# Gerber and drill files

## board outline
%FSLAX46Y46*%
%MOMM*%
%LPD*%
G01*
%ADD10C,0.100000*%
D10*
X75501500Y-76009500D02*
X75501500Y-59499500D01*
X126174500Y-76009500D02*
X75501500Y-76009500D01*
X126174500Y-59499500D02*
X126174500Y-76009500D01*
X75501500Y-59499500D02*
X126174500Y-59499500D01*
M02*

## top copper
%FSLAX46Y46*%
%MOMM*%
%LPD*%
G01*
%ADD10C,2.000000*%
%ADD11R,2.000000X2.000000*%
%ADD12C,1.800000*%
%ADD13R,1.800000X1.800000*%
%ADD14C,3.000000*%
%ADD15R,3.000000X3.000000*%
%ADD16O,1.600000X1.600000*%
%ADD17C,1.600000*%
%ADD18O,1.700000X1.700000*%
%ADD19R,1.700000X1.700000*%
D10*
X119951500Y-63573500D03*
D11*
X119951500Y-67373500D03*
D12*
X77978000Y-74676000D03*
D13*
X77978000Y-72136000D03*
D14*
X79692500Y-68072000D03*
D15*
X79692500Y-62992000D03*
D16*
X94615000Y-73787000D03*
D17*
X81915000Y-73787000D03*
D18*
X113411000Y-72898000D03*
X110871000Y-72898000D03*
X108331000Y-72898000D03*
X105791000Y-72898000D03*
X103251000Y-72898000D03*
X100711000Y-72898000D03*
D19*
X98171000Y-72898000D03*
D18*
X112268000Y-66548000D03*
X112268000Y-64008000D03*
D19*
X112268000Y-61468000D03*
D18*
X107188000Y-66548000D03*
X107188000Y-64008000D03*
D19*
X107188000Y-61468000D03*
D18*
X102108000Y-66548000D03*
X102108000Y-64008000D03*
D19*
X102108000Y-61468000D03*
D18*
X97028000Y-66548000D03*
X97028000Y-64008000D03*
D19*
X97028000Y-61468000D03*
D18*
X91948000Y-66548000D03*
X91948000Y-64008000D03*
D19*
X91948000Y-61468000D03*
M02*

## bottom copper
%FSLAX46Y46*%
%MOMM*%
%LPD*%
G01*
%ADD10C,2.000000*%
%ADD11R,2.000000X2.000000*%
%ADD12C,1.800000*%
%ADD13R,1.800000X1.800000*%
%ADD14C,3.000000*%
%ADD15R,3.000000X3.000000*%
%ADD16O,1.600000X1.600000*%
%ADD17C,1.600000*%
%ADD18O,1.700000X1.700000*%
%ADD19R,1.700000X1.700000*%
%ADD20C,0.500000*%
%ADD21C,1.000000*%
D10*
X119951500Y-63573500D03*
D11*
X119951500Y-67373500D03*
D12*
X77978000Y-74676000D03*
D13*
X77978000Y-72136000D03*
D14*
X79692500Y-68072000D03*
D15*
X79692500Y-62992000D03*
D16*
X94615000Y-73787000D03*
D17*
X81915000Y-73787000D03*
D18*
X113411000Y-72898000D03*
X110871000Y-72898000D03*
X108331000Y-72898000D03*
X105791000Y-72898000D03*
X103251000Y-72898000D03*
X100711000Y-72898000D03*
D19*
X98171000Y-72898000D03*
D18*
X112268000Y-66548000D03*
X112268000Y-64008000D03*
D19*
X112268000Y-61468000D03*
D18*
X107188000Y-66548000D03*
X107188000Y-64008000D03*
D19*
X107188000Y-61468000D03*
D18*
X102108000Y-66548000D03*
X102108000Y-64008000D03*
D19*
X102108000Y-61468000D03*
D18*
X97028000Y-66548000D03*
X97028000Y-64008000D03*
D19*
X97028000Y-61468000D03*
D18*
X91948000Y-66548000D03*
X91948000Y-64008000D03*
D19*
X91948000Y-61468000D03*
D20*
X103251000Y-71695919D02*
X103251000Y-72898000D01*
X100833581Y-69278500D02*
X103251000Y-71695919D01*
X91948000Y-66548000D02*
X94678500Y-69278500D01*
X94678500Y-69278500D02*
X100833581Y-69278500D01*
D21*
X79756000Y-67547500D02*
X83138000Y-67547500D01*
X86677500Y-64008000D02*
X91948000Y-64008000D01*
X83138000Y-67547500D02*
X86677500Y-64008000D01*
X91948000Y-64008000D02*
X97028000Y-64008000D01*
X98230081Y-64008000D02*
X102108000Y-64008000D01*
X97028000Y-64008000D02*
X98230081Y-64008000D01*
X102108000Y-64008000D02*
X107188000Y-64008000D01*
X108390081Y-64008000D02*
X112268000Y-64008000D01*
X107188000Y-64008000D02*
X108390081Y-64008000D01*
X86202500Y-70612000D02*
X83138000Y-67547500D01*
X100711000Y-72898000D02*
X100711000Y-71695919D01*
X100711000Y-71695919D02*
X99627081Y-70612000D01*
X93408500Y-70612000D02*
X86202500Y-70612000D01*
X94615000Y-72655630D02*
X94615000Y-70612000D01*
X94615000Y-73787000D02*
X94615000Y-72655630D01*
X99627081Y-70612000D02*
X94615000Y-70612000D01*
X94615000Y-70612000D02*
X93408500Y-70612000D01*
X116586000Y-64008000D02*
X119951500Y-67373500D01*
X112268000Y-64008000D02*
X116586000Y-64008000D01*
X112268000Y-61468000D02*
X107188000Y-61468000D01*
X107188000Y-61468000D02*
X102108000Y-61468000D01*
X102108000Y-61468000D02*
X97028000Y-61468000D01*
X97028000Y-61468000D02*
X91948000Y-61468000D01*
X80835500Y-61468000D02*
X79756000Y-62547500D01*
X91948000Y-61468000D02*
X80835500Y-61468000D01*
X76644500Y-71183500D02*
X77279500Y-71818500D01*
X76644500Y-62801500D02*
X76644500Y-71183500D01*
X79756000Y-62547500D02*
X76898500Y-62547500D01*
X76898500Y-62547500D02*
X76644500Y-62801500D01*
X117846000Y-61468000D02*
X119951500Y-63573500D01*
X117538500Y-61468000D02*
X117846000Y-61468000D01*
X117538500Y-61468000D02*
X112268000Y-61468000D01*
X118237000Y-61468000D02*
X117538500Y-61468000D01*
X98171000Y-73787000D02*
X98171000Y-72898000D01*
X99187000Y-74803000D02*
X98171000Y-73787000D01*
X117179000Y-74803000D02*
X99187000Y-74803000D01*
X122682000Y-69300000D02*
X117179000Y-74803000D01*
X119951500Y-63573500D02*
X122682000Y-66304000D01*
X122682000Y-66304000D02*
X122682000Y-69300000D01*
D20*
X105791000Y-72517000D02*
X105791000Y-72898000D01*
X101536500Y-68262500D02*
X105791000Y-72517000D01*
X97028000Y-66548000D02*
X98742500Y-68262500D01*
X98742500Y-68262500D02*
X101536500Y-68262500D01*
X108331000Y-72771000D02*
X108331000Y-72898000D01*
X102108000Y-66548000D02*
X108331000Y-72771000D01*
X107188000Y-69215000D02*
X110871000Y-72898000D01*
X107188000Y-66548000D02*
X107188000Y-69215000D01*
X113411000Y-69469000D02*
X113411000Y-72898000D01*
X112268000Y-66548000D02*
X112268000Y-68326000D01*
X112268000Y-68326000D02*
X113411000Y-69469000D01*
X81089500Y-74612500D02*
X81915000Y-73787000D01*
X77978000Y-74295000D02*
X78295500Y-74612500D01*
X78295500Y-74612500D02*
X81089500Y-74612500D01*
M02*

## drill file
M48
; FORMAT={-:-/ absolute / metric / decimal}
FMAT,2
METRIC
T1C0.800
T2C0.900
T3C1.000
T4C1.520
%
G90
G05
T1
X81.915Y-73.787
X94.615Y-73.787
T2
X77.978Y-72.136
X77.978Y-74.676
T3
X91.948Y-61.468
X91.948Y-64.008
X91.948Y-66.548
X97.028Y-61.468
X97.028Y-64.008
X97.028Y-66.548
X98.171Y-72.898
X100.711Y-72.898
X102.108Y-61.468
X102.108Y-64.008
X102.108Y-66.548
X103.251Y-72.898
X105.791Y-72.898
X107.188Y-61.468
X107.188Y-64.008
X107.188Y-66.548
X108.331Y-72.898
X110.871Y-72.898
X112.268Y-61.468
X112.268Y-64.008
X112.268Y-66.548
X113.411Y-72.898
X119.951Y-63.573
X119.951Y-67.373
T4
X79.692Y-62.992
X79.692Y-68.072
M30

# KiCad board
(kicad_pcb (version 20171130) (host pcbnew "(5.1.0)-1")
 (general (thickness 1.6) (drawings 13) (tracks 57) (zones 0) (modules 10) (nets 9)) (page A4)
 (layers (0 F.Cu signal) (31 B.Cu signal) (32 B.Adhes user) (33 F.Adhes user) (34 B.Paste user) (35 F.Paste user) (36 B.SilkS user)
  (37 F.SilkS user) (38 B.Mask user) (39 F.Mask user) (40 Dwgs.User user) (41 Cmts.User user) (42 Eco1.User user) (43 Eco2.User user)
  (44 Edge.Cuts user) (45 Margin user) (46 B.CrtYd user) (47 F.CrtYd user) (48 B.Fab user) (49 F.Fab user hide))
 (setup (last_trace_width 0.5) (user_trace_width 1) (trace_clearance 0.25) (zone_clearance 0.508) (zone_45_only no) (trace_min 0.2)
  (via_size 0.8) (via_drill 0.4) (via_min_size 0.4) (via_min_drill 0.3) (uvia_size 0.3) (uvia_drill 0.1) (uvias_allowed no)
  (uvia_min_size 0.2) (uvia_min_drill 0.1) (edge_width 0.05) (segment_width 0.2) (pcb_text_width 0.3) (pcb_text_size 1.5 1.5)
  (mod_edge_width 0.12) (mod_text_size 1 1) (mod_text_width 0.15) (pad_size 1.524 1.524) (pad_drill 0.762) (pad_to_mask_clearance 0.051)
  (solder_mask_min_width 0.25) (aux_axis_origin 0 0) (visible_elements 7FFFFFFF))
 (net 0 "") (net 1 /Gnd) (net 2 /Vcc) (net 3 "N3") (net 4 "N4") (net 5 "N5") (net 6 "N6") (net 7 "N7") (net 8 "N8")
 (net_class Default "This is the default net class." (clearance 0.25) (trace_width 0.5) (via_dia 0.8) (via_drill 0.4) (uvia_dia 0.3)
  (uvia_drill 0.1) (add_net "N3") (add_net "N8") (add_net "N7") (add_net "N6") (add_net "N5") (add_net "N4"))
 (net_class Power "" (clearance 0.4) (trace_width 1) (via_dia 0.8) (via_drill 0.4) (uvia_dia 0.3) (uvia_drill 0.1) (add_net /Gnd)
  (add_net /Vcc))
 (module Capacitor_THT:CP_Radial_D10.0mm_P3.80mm (layer F.Cu) (at 119.9515 67.3735 90)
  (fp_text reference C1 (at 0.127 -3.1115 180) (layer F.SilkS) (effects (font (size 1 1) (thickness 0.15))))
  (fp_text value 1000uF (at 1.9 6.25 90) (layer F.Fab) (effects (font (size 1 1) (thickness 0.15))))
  (pad 2 thru_hole circle (at 3.8 0 90) (size 2 2) (drill 1) (layers *.Cu *.Mask) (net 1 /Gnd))
  (pad 1 thru_hole rect (at 0 0 90) (size 2 2) (drill 1) (layers *.Cu *.Mask) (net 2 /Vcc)))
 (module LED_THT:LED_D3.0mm (layer F.Cu) (at 77.978 72.136 270)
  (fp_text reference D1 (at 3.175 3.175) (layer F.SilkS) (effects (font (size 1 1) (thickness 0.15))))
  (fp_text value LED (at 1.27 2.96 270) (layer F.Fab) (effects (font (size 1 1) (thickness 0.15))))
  (pad 2 thru_hole circle (at 2.54 0 270) (size 1.8 1.8) (drill 0.9) (layers *.Cu *.Mask) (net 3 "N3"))
  (pad 1 thru_hole rect (at 0 0 270) (size 1.8 1.8) (drill 0.9) (layers *.Cu *.Mask) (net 1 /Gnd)))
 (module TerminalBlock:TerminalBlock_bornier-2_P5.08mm (layer F.Cu) (at 79.6925 62.992 270)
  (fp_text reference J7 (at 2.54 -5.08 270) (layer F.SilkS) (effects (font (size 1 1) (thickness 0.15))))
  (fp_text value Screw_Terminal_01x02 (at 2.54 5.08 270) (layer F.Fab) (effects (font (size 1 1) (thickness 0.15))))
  (pad 2 thru_hole circle (at 5.08 0 270) (size 3 3) (drill 1.52) (layers *.Cu *.Mask) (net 2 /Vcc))
  (pad 1 thru_hole rect (at 0 0 270) (size 3 3) (drill 1.52) (layers *.Cu *.Mask) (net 1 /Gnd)))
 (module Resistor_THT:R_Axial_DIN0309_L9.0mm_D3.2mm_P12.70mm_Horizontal (layer F.Cu) (at 81.915 73.787)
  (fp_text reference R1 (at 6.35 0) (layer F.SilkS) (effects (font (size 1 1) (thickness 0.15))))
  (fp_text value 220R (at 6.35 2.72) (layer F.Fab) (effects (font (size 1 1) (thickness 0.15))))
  (pad 2 thru_hole oval (at 12.7 0) (size 1.6 1.6) (drill 0.8) (layers *.Cu *.Mask) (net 2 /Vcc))
  (pad 1 thru_hole circle (at 0 0) (size 1.6 1.6) (drill 0.8) (layers *.Cu *.Mask) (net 3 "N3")))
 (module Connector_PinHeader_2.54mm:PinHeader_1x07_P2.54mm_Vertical (layer F.Cu) (at 98.171 72.898 90)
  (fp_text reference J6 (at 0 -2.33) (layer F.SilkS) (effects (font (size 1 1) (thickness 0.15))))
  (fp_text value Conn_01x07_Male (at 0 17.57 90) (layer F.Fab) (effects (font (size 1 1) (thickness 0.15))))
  (pad 7 thru_hole oval (at 0 15.24 90) (size 1.7 1.7) (drill 1) (layers *.Cu *.Mask) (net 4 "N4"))
  (pad 6 thru_hole oval (at 0 12.7 90) (size 1.7 1.7) (drill 1) (layers *.Cu *.Mask) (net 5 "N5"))
  (pad 5 thru_hole oval (at 0 10.16 90) (size 1.7 1.7) (drill 1) (layers *.Cu *.Mask) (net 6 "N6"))
  (pad 4 thru_hole oval (at 0 7.62 90) (size 1.7 1.7) (drill 1) (layers *.Cu *.Mask) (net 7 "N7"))
  (pad 3 thru_hole oval (at 0 5.08 90) (size 1.7 1.7) (drill 1) (layers *.Cu *.Mask) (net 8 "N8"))
  (pad 2 thru_hole oval (at 0 2.54 90) (size 1.7 1.7) (drill 1) (layers *.Cu *.Mask) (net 2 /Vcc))
  (pad 1 thru_hole rect (at 0 0 90) (size 1.7 1.7) (drill 1) (layers *.Cu *.Mask) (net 1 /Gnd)))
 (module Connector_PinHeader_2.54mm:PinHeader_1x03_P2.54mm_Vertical (layer F.Cu) (at 112.268 61.468)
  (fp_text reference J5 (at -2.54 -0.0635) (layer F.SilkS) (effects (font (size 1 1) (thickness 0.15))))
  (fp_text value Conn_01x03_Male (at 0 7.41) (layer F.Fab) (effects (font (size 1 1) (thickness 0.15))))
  (pad 3 thru_hole oval (at 0 5.08) (size 1.7 1.7) (drill 1) (layers *.Cu *.Mask) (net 4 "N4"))
  (pad 2 thru_hole oval (at 0 2.54) (size 1.7 1.7) (drill 1) (layers *.Cu *.Mask) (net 2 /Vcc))
  (pad 1 thru_hole rect (at 0 0) (size 1.7 1.7) (drill 1) (layers *.Cu *.Mask) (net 1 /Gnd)))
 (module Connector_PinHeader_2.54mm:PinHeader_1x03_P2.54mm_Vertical (layer F.Cu) (at 107.188 61.468)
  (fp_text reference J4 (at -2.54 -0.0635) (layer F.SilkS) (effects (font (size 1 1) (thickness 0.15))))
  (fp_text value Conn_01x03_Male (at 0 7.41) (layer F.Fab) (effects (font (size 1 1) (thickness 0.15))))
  (pad 3 thru_hole oval (at 0 5.08) (size 1.7 1.7) (drill 1) (layers *.Cu *.Mask) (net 5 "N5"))
  (pad 2 thru_hole oval (at 0 2.54) (size 1.7 1.7) (drill 1) (layers *.Cu *.Mask) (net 2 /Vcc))
  (pad 1 thru_hole rect (at 0 0) (size 1.7 1.7) (drill 1) (layers *.Cu *.Mask) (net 1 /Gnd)))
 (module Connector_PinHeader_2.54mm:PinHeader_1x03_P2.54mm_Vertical (layer F.Cu) (at 102.108 61.468)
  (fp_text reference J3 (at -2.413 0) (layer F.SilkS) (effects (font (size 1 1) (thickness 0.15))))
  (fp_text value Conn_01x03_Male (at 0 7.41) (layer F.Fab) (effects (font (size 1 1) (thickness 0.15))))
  (pad 3 thru_hole oval (at 0 5.08) (size 1.7 1.7) (drill 1) (layers *.Cu *.Mask) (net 6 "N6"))
  (pad 2 thru_hole oval (at 0 2.54) (size 1.7 1.7) (drill 1) (layers *.Cu *.Mask) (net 2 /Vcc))
  (pad 1 thru_hole rect (at 0 0) (size 1.7 1.7) (drill 1) (layers *.Cu *.Mask) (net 1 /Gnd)))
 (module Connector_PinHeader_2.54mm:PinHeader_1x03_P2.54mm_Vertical (layer F.Cu) (at 97.028 61.468)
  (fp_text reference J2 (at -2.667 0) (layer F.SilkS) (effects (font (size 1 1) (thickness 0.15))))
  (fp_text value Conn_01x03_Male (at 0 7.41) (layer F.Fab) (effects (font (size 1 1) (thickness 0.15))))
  (pad 3 thru_hole oval (at 0 5.08) (size 1.7 1.7) (drill 1) (layers *.Cu *.Mask) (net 7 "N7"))
  (pad 2 thru_hole oval (at 0 2.54) (size 1.7 1.7) (drill 1) (layers *.Cu *.Mask) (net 2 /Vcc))
  (pad 1 thru_hole rect (at 0 0) (size 1.7 1.7) (drill 1) (layers *.Cu *.Mask) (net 1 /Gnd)))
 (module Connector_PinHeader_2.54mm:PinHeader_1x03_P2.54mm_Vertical (layer F.Cu) (at 91.948 61.468)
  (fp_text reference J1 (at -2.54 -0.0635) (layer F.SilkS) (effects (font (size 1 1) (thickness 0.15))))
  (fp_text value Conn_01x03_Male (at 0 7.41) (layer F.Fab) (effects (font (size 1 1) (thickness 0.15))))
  (pad 3 thru_hole oval (at 0 5.08) (size 1.7 1.7) (drill 1) (layers *.Cu *.Mask) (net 8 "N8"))
  (pad 2 thru_hole oval (at 0 2.54) (size 1.7 1.7) (drill 1) (layers *.Cu *.Mask) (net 2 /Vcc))
  (pad 1 thru_hole rect (at 0 0) (size 1.7 1.7) (drill 1) (layers *.Cu *.Mask) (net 1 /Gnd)))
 (gr_line (start 75.5015 76.0095) (end 75.5015 59.4995) (layer Edge.Cuts) (width 0.1))
 (gr_line (start 126.1745 76.0095) (end 75.5015 76.0095) (layer Edge.Cuts) (width 0.1))
 (gr_line (start 126.1745 59.4995) (end 126.1745 76.0095) (layer Edge.Cuts) (width 0.1))
 (gr_line (start 75.5015 59.4995) (end 126.1745 59.4995) (layer Edge.Cuts) (width 0.1))
 (segment (start 103.251 71.695919) (end 103.251 72.898) (width 0.5) (layer B.Cu) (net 8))
 (segment (start 100.833581 69.2785) (end 103.251 71.695919) (width 0.5) (layer B.Cu) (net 8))
 (segment (start 91.948 66.548) (end 94.6785 69.2785) (width 0.5) (layer B.Cu) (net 8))
 (segment (start 94.6785 69.2785) (end 100.833581 69.2785) (width 0.5) (layer B.Cu) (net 8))
 (segment (start 79.756 67.5475) (end 83.138 67.5475) (width 1) (layer B.Cu) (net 2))
 (segment (start 86.6775 64.008) (end 91.948 64.008) (width 1) (layer B.Cu) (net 2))
 (segment (start 83.138 67.5475) (end 86.6775 64.008) (width 1) (layer B.Cu) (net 2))
 (segment (start 91.948 64.008) (end 97.028 64.008) (width 1) (layer B.Cu) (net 2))
 (segment (start 98.230081 64.008) (end 102.108 64.008) (width 1) (layer B.Cu) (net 2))
 (segment (start 97.028 64.008) (end 98.230081 64.008) (width 1) (layer B.Cu) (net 2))
 (segment (start 102.108 64.008) (end 107.188 64.008) (width 1) (layer B.Cu) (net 2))
 (segment (start 108.390081 64.008) (end 112.268 64.008) (width 1) (layer B.Cu) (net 2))
 (segment (start 107.188 64.008) (end 108.390081 64.008) (width 1) (layer B.Cu) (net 2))
 (segment (start 86.2025 70.612) (end 83.138 67.5475) (width 1) (layer B.Cu) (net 2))
 (segment (start 100.711 72.898) (end 100.711 71.695919) (width 1) (layer B.Cu) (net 2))
 (segment (start 100.711 71.695919) (end 99.627081 70.612) (width 1) (layer B.Cu) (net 2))
 (segment (start 93.4085 70.612) (end 86.2025 70.612) (width 1) (layer B.Cu) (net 2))
 (segment (start 94.615 72.65563) (end 94.615 70.612) (width 1) (layer B.Cu) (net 2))
 (segment (start 94.615 73.787) (end 94.615 72.65563) (width 1) (layer B.Cu) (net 2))
 (segment (start 99.627081 70.612) (end 94.615 70.612) (width 1) (layer B.Cu) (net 2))
 (segment (start 94.615 70.612) (end 93.4085 70.612) (width 1) (layer B.Cu) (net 2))
 (segment (start 116.586 64.008) (end 119.9515 67.3735) (width 1) (layer B.Cu) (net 2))
 (segment (start 112.268 64.008) (end 116.586 64.008) (width 1) (layer B.Cu) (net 2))
 (segment (start 112.268 61.468) (end 107.188 61.468) (width 1) (layer B.Cu) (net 1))
 (segment (start 107.188 61.468) (end 102.108 61.468) (width 1) (layer B.Cu) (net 1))
 (segment (start 102.108 61.468) (end 97.028 61.468) (width 1) (layer B.Cu) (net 1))
 (segment (start 97.028 61.468) (end 91.948 61.468) (width 1) (layer B.Cu) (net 1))
 (segment (start 80.8355 61.468) (end 79.756 62.5475) (width 1) (layer B.Cu) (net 1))
 (segment (start 91.948 61.468) (end 80.8355 61.468) (width 1) (layer B.Cu) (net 1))
 (segment (start 76.6445 71.1835) (end 77.2795 71.8185) (width 1) (layer B.Cu) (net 1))
 (segment (start 76.6445 62.8015) (end 76.6445 71.1835) (width 1) (layer B.Cu) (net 1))
 (segment (start 79.756 62.5475) (end 76.8985 62.5475) (width 1) (layer B.Cu) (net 1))
 (segment (start 76.8985 62.5475) (end 76.6445 62.8015) (width 1) (layer B.Cu) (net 1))
 (segment (start 117.846 61.468) (end 119.9515 63.5735) (width 1) (layer B.Cu) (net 1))
 (segment (start 117.5385 61.468) (end 117.846 61.468) (width 1) (layer B.Cu) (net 1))
 (segment (start 117.5385 61.468) (end 112.268 61.468) (width 1) (layer B.Cu) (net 1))
 (segment (start 118.237 61.468) (end 117.5385 61.468) (width 1) (layer B.Cu) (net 1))
 (segment (start 98.171 73.787) (end 98.171 72.898) (width 1) (layer B.Cu) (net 1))
 (segment (start 99.187 74.803) (end 98.171 73.787) (width 1) (layer B.Cu) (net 1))
 (segment (start 117.179 74.803) (end 99.187 74.803) (width 1) (layer B.Cu) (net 1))
 (segment (start 122.682 69.3) (end 117.179 74.803) (width 1) (layer B.Cu) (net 1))
 (segment (start 119.9515 63.5735) (end 122.682 66.304) (width 1) (layer B.Cu) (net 1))
 (segment (start 122.682 66.304) (end 122.682 69.3) (width 1) (layer B.Cu) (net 1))
 (segment (start 105.791 72.517) (end 105.791 72.898) (width 0.5) (layer B.Cu) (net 7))
 (segment (start 101.5365 68.2625) (end 105.791 72.517) (width 0.5) (layer B.Cu) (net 7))
 (segment (start 97.028 66.548) (end 98.7425 68.2625) (width 0.5) (layer B.Cu) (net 7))
 (segment (start 98.7425 68.2625) (end 101.5365 68.2625) (width 0.5) (layer B.Cu) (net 7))
 (segment (start 108.331 72.771) (end 108.331 72.898) (width 0.5) (layer B.Cu) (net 6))
 (segment (start 102.108 66.548) (end 108.331 72.771) (width 0.5) (layer B.Cu) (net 6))
 (segment (start 107.188 69.215) (end 110.871 72.898) (width 0.5) (layer B.Cu) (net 5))
 (segment (start 107.188 66.548) (end 107.188 69.215) (width 0.5) (layer B.Cu) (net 5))
 (segment (start 113.411 69.469) (end 113.411 72.898) (width 0.5) (layer B.Cu) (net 4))
 (segment (start 112.268 66.548) (end 112.268 68.326) (width 0.5) (layer B.Cu) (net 4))
 (segment (start 112.268 68.326) (end 113.411 69.469) (width 0.5) (layer B.Cu) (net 4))
 (segment (start 81.0895 74.6125) (end 81.915 73.787) (width 0.5) (layer B.Cu) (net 3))
 (segment (start 77.978 74.295) (end 78.2955 74.6125) (width 0.5) (layer B.Cu) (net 3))
 (segment (start 78.2955 74.6125) (end 81.0895 74.6125) (width 0.5) (layer B.Cu) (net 3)))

